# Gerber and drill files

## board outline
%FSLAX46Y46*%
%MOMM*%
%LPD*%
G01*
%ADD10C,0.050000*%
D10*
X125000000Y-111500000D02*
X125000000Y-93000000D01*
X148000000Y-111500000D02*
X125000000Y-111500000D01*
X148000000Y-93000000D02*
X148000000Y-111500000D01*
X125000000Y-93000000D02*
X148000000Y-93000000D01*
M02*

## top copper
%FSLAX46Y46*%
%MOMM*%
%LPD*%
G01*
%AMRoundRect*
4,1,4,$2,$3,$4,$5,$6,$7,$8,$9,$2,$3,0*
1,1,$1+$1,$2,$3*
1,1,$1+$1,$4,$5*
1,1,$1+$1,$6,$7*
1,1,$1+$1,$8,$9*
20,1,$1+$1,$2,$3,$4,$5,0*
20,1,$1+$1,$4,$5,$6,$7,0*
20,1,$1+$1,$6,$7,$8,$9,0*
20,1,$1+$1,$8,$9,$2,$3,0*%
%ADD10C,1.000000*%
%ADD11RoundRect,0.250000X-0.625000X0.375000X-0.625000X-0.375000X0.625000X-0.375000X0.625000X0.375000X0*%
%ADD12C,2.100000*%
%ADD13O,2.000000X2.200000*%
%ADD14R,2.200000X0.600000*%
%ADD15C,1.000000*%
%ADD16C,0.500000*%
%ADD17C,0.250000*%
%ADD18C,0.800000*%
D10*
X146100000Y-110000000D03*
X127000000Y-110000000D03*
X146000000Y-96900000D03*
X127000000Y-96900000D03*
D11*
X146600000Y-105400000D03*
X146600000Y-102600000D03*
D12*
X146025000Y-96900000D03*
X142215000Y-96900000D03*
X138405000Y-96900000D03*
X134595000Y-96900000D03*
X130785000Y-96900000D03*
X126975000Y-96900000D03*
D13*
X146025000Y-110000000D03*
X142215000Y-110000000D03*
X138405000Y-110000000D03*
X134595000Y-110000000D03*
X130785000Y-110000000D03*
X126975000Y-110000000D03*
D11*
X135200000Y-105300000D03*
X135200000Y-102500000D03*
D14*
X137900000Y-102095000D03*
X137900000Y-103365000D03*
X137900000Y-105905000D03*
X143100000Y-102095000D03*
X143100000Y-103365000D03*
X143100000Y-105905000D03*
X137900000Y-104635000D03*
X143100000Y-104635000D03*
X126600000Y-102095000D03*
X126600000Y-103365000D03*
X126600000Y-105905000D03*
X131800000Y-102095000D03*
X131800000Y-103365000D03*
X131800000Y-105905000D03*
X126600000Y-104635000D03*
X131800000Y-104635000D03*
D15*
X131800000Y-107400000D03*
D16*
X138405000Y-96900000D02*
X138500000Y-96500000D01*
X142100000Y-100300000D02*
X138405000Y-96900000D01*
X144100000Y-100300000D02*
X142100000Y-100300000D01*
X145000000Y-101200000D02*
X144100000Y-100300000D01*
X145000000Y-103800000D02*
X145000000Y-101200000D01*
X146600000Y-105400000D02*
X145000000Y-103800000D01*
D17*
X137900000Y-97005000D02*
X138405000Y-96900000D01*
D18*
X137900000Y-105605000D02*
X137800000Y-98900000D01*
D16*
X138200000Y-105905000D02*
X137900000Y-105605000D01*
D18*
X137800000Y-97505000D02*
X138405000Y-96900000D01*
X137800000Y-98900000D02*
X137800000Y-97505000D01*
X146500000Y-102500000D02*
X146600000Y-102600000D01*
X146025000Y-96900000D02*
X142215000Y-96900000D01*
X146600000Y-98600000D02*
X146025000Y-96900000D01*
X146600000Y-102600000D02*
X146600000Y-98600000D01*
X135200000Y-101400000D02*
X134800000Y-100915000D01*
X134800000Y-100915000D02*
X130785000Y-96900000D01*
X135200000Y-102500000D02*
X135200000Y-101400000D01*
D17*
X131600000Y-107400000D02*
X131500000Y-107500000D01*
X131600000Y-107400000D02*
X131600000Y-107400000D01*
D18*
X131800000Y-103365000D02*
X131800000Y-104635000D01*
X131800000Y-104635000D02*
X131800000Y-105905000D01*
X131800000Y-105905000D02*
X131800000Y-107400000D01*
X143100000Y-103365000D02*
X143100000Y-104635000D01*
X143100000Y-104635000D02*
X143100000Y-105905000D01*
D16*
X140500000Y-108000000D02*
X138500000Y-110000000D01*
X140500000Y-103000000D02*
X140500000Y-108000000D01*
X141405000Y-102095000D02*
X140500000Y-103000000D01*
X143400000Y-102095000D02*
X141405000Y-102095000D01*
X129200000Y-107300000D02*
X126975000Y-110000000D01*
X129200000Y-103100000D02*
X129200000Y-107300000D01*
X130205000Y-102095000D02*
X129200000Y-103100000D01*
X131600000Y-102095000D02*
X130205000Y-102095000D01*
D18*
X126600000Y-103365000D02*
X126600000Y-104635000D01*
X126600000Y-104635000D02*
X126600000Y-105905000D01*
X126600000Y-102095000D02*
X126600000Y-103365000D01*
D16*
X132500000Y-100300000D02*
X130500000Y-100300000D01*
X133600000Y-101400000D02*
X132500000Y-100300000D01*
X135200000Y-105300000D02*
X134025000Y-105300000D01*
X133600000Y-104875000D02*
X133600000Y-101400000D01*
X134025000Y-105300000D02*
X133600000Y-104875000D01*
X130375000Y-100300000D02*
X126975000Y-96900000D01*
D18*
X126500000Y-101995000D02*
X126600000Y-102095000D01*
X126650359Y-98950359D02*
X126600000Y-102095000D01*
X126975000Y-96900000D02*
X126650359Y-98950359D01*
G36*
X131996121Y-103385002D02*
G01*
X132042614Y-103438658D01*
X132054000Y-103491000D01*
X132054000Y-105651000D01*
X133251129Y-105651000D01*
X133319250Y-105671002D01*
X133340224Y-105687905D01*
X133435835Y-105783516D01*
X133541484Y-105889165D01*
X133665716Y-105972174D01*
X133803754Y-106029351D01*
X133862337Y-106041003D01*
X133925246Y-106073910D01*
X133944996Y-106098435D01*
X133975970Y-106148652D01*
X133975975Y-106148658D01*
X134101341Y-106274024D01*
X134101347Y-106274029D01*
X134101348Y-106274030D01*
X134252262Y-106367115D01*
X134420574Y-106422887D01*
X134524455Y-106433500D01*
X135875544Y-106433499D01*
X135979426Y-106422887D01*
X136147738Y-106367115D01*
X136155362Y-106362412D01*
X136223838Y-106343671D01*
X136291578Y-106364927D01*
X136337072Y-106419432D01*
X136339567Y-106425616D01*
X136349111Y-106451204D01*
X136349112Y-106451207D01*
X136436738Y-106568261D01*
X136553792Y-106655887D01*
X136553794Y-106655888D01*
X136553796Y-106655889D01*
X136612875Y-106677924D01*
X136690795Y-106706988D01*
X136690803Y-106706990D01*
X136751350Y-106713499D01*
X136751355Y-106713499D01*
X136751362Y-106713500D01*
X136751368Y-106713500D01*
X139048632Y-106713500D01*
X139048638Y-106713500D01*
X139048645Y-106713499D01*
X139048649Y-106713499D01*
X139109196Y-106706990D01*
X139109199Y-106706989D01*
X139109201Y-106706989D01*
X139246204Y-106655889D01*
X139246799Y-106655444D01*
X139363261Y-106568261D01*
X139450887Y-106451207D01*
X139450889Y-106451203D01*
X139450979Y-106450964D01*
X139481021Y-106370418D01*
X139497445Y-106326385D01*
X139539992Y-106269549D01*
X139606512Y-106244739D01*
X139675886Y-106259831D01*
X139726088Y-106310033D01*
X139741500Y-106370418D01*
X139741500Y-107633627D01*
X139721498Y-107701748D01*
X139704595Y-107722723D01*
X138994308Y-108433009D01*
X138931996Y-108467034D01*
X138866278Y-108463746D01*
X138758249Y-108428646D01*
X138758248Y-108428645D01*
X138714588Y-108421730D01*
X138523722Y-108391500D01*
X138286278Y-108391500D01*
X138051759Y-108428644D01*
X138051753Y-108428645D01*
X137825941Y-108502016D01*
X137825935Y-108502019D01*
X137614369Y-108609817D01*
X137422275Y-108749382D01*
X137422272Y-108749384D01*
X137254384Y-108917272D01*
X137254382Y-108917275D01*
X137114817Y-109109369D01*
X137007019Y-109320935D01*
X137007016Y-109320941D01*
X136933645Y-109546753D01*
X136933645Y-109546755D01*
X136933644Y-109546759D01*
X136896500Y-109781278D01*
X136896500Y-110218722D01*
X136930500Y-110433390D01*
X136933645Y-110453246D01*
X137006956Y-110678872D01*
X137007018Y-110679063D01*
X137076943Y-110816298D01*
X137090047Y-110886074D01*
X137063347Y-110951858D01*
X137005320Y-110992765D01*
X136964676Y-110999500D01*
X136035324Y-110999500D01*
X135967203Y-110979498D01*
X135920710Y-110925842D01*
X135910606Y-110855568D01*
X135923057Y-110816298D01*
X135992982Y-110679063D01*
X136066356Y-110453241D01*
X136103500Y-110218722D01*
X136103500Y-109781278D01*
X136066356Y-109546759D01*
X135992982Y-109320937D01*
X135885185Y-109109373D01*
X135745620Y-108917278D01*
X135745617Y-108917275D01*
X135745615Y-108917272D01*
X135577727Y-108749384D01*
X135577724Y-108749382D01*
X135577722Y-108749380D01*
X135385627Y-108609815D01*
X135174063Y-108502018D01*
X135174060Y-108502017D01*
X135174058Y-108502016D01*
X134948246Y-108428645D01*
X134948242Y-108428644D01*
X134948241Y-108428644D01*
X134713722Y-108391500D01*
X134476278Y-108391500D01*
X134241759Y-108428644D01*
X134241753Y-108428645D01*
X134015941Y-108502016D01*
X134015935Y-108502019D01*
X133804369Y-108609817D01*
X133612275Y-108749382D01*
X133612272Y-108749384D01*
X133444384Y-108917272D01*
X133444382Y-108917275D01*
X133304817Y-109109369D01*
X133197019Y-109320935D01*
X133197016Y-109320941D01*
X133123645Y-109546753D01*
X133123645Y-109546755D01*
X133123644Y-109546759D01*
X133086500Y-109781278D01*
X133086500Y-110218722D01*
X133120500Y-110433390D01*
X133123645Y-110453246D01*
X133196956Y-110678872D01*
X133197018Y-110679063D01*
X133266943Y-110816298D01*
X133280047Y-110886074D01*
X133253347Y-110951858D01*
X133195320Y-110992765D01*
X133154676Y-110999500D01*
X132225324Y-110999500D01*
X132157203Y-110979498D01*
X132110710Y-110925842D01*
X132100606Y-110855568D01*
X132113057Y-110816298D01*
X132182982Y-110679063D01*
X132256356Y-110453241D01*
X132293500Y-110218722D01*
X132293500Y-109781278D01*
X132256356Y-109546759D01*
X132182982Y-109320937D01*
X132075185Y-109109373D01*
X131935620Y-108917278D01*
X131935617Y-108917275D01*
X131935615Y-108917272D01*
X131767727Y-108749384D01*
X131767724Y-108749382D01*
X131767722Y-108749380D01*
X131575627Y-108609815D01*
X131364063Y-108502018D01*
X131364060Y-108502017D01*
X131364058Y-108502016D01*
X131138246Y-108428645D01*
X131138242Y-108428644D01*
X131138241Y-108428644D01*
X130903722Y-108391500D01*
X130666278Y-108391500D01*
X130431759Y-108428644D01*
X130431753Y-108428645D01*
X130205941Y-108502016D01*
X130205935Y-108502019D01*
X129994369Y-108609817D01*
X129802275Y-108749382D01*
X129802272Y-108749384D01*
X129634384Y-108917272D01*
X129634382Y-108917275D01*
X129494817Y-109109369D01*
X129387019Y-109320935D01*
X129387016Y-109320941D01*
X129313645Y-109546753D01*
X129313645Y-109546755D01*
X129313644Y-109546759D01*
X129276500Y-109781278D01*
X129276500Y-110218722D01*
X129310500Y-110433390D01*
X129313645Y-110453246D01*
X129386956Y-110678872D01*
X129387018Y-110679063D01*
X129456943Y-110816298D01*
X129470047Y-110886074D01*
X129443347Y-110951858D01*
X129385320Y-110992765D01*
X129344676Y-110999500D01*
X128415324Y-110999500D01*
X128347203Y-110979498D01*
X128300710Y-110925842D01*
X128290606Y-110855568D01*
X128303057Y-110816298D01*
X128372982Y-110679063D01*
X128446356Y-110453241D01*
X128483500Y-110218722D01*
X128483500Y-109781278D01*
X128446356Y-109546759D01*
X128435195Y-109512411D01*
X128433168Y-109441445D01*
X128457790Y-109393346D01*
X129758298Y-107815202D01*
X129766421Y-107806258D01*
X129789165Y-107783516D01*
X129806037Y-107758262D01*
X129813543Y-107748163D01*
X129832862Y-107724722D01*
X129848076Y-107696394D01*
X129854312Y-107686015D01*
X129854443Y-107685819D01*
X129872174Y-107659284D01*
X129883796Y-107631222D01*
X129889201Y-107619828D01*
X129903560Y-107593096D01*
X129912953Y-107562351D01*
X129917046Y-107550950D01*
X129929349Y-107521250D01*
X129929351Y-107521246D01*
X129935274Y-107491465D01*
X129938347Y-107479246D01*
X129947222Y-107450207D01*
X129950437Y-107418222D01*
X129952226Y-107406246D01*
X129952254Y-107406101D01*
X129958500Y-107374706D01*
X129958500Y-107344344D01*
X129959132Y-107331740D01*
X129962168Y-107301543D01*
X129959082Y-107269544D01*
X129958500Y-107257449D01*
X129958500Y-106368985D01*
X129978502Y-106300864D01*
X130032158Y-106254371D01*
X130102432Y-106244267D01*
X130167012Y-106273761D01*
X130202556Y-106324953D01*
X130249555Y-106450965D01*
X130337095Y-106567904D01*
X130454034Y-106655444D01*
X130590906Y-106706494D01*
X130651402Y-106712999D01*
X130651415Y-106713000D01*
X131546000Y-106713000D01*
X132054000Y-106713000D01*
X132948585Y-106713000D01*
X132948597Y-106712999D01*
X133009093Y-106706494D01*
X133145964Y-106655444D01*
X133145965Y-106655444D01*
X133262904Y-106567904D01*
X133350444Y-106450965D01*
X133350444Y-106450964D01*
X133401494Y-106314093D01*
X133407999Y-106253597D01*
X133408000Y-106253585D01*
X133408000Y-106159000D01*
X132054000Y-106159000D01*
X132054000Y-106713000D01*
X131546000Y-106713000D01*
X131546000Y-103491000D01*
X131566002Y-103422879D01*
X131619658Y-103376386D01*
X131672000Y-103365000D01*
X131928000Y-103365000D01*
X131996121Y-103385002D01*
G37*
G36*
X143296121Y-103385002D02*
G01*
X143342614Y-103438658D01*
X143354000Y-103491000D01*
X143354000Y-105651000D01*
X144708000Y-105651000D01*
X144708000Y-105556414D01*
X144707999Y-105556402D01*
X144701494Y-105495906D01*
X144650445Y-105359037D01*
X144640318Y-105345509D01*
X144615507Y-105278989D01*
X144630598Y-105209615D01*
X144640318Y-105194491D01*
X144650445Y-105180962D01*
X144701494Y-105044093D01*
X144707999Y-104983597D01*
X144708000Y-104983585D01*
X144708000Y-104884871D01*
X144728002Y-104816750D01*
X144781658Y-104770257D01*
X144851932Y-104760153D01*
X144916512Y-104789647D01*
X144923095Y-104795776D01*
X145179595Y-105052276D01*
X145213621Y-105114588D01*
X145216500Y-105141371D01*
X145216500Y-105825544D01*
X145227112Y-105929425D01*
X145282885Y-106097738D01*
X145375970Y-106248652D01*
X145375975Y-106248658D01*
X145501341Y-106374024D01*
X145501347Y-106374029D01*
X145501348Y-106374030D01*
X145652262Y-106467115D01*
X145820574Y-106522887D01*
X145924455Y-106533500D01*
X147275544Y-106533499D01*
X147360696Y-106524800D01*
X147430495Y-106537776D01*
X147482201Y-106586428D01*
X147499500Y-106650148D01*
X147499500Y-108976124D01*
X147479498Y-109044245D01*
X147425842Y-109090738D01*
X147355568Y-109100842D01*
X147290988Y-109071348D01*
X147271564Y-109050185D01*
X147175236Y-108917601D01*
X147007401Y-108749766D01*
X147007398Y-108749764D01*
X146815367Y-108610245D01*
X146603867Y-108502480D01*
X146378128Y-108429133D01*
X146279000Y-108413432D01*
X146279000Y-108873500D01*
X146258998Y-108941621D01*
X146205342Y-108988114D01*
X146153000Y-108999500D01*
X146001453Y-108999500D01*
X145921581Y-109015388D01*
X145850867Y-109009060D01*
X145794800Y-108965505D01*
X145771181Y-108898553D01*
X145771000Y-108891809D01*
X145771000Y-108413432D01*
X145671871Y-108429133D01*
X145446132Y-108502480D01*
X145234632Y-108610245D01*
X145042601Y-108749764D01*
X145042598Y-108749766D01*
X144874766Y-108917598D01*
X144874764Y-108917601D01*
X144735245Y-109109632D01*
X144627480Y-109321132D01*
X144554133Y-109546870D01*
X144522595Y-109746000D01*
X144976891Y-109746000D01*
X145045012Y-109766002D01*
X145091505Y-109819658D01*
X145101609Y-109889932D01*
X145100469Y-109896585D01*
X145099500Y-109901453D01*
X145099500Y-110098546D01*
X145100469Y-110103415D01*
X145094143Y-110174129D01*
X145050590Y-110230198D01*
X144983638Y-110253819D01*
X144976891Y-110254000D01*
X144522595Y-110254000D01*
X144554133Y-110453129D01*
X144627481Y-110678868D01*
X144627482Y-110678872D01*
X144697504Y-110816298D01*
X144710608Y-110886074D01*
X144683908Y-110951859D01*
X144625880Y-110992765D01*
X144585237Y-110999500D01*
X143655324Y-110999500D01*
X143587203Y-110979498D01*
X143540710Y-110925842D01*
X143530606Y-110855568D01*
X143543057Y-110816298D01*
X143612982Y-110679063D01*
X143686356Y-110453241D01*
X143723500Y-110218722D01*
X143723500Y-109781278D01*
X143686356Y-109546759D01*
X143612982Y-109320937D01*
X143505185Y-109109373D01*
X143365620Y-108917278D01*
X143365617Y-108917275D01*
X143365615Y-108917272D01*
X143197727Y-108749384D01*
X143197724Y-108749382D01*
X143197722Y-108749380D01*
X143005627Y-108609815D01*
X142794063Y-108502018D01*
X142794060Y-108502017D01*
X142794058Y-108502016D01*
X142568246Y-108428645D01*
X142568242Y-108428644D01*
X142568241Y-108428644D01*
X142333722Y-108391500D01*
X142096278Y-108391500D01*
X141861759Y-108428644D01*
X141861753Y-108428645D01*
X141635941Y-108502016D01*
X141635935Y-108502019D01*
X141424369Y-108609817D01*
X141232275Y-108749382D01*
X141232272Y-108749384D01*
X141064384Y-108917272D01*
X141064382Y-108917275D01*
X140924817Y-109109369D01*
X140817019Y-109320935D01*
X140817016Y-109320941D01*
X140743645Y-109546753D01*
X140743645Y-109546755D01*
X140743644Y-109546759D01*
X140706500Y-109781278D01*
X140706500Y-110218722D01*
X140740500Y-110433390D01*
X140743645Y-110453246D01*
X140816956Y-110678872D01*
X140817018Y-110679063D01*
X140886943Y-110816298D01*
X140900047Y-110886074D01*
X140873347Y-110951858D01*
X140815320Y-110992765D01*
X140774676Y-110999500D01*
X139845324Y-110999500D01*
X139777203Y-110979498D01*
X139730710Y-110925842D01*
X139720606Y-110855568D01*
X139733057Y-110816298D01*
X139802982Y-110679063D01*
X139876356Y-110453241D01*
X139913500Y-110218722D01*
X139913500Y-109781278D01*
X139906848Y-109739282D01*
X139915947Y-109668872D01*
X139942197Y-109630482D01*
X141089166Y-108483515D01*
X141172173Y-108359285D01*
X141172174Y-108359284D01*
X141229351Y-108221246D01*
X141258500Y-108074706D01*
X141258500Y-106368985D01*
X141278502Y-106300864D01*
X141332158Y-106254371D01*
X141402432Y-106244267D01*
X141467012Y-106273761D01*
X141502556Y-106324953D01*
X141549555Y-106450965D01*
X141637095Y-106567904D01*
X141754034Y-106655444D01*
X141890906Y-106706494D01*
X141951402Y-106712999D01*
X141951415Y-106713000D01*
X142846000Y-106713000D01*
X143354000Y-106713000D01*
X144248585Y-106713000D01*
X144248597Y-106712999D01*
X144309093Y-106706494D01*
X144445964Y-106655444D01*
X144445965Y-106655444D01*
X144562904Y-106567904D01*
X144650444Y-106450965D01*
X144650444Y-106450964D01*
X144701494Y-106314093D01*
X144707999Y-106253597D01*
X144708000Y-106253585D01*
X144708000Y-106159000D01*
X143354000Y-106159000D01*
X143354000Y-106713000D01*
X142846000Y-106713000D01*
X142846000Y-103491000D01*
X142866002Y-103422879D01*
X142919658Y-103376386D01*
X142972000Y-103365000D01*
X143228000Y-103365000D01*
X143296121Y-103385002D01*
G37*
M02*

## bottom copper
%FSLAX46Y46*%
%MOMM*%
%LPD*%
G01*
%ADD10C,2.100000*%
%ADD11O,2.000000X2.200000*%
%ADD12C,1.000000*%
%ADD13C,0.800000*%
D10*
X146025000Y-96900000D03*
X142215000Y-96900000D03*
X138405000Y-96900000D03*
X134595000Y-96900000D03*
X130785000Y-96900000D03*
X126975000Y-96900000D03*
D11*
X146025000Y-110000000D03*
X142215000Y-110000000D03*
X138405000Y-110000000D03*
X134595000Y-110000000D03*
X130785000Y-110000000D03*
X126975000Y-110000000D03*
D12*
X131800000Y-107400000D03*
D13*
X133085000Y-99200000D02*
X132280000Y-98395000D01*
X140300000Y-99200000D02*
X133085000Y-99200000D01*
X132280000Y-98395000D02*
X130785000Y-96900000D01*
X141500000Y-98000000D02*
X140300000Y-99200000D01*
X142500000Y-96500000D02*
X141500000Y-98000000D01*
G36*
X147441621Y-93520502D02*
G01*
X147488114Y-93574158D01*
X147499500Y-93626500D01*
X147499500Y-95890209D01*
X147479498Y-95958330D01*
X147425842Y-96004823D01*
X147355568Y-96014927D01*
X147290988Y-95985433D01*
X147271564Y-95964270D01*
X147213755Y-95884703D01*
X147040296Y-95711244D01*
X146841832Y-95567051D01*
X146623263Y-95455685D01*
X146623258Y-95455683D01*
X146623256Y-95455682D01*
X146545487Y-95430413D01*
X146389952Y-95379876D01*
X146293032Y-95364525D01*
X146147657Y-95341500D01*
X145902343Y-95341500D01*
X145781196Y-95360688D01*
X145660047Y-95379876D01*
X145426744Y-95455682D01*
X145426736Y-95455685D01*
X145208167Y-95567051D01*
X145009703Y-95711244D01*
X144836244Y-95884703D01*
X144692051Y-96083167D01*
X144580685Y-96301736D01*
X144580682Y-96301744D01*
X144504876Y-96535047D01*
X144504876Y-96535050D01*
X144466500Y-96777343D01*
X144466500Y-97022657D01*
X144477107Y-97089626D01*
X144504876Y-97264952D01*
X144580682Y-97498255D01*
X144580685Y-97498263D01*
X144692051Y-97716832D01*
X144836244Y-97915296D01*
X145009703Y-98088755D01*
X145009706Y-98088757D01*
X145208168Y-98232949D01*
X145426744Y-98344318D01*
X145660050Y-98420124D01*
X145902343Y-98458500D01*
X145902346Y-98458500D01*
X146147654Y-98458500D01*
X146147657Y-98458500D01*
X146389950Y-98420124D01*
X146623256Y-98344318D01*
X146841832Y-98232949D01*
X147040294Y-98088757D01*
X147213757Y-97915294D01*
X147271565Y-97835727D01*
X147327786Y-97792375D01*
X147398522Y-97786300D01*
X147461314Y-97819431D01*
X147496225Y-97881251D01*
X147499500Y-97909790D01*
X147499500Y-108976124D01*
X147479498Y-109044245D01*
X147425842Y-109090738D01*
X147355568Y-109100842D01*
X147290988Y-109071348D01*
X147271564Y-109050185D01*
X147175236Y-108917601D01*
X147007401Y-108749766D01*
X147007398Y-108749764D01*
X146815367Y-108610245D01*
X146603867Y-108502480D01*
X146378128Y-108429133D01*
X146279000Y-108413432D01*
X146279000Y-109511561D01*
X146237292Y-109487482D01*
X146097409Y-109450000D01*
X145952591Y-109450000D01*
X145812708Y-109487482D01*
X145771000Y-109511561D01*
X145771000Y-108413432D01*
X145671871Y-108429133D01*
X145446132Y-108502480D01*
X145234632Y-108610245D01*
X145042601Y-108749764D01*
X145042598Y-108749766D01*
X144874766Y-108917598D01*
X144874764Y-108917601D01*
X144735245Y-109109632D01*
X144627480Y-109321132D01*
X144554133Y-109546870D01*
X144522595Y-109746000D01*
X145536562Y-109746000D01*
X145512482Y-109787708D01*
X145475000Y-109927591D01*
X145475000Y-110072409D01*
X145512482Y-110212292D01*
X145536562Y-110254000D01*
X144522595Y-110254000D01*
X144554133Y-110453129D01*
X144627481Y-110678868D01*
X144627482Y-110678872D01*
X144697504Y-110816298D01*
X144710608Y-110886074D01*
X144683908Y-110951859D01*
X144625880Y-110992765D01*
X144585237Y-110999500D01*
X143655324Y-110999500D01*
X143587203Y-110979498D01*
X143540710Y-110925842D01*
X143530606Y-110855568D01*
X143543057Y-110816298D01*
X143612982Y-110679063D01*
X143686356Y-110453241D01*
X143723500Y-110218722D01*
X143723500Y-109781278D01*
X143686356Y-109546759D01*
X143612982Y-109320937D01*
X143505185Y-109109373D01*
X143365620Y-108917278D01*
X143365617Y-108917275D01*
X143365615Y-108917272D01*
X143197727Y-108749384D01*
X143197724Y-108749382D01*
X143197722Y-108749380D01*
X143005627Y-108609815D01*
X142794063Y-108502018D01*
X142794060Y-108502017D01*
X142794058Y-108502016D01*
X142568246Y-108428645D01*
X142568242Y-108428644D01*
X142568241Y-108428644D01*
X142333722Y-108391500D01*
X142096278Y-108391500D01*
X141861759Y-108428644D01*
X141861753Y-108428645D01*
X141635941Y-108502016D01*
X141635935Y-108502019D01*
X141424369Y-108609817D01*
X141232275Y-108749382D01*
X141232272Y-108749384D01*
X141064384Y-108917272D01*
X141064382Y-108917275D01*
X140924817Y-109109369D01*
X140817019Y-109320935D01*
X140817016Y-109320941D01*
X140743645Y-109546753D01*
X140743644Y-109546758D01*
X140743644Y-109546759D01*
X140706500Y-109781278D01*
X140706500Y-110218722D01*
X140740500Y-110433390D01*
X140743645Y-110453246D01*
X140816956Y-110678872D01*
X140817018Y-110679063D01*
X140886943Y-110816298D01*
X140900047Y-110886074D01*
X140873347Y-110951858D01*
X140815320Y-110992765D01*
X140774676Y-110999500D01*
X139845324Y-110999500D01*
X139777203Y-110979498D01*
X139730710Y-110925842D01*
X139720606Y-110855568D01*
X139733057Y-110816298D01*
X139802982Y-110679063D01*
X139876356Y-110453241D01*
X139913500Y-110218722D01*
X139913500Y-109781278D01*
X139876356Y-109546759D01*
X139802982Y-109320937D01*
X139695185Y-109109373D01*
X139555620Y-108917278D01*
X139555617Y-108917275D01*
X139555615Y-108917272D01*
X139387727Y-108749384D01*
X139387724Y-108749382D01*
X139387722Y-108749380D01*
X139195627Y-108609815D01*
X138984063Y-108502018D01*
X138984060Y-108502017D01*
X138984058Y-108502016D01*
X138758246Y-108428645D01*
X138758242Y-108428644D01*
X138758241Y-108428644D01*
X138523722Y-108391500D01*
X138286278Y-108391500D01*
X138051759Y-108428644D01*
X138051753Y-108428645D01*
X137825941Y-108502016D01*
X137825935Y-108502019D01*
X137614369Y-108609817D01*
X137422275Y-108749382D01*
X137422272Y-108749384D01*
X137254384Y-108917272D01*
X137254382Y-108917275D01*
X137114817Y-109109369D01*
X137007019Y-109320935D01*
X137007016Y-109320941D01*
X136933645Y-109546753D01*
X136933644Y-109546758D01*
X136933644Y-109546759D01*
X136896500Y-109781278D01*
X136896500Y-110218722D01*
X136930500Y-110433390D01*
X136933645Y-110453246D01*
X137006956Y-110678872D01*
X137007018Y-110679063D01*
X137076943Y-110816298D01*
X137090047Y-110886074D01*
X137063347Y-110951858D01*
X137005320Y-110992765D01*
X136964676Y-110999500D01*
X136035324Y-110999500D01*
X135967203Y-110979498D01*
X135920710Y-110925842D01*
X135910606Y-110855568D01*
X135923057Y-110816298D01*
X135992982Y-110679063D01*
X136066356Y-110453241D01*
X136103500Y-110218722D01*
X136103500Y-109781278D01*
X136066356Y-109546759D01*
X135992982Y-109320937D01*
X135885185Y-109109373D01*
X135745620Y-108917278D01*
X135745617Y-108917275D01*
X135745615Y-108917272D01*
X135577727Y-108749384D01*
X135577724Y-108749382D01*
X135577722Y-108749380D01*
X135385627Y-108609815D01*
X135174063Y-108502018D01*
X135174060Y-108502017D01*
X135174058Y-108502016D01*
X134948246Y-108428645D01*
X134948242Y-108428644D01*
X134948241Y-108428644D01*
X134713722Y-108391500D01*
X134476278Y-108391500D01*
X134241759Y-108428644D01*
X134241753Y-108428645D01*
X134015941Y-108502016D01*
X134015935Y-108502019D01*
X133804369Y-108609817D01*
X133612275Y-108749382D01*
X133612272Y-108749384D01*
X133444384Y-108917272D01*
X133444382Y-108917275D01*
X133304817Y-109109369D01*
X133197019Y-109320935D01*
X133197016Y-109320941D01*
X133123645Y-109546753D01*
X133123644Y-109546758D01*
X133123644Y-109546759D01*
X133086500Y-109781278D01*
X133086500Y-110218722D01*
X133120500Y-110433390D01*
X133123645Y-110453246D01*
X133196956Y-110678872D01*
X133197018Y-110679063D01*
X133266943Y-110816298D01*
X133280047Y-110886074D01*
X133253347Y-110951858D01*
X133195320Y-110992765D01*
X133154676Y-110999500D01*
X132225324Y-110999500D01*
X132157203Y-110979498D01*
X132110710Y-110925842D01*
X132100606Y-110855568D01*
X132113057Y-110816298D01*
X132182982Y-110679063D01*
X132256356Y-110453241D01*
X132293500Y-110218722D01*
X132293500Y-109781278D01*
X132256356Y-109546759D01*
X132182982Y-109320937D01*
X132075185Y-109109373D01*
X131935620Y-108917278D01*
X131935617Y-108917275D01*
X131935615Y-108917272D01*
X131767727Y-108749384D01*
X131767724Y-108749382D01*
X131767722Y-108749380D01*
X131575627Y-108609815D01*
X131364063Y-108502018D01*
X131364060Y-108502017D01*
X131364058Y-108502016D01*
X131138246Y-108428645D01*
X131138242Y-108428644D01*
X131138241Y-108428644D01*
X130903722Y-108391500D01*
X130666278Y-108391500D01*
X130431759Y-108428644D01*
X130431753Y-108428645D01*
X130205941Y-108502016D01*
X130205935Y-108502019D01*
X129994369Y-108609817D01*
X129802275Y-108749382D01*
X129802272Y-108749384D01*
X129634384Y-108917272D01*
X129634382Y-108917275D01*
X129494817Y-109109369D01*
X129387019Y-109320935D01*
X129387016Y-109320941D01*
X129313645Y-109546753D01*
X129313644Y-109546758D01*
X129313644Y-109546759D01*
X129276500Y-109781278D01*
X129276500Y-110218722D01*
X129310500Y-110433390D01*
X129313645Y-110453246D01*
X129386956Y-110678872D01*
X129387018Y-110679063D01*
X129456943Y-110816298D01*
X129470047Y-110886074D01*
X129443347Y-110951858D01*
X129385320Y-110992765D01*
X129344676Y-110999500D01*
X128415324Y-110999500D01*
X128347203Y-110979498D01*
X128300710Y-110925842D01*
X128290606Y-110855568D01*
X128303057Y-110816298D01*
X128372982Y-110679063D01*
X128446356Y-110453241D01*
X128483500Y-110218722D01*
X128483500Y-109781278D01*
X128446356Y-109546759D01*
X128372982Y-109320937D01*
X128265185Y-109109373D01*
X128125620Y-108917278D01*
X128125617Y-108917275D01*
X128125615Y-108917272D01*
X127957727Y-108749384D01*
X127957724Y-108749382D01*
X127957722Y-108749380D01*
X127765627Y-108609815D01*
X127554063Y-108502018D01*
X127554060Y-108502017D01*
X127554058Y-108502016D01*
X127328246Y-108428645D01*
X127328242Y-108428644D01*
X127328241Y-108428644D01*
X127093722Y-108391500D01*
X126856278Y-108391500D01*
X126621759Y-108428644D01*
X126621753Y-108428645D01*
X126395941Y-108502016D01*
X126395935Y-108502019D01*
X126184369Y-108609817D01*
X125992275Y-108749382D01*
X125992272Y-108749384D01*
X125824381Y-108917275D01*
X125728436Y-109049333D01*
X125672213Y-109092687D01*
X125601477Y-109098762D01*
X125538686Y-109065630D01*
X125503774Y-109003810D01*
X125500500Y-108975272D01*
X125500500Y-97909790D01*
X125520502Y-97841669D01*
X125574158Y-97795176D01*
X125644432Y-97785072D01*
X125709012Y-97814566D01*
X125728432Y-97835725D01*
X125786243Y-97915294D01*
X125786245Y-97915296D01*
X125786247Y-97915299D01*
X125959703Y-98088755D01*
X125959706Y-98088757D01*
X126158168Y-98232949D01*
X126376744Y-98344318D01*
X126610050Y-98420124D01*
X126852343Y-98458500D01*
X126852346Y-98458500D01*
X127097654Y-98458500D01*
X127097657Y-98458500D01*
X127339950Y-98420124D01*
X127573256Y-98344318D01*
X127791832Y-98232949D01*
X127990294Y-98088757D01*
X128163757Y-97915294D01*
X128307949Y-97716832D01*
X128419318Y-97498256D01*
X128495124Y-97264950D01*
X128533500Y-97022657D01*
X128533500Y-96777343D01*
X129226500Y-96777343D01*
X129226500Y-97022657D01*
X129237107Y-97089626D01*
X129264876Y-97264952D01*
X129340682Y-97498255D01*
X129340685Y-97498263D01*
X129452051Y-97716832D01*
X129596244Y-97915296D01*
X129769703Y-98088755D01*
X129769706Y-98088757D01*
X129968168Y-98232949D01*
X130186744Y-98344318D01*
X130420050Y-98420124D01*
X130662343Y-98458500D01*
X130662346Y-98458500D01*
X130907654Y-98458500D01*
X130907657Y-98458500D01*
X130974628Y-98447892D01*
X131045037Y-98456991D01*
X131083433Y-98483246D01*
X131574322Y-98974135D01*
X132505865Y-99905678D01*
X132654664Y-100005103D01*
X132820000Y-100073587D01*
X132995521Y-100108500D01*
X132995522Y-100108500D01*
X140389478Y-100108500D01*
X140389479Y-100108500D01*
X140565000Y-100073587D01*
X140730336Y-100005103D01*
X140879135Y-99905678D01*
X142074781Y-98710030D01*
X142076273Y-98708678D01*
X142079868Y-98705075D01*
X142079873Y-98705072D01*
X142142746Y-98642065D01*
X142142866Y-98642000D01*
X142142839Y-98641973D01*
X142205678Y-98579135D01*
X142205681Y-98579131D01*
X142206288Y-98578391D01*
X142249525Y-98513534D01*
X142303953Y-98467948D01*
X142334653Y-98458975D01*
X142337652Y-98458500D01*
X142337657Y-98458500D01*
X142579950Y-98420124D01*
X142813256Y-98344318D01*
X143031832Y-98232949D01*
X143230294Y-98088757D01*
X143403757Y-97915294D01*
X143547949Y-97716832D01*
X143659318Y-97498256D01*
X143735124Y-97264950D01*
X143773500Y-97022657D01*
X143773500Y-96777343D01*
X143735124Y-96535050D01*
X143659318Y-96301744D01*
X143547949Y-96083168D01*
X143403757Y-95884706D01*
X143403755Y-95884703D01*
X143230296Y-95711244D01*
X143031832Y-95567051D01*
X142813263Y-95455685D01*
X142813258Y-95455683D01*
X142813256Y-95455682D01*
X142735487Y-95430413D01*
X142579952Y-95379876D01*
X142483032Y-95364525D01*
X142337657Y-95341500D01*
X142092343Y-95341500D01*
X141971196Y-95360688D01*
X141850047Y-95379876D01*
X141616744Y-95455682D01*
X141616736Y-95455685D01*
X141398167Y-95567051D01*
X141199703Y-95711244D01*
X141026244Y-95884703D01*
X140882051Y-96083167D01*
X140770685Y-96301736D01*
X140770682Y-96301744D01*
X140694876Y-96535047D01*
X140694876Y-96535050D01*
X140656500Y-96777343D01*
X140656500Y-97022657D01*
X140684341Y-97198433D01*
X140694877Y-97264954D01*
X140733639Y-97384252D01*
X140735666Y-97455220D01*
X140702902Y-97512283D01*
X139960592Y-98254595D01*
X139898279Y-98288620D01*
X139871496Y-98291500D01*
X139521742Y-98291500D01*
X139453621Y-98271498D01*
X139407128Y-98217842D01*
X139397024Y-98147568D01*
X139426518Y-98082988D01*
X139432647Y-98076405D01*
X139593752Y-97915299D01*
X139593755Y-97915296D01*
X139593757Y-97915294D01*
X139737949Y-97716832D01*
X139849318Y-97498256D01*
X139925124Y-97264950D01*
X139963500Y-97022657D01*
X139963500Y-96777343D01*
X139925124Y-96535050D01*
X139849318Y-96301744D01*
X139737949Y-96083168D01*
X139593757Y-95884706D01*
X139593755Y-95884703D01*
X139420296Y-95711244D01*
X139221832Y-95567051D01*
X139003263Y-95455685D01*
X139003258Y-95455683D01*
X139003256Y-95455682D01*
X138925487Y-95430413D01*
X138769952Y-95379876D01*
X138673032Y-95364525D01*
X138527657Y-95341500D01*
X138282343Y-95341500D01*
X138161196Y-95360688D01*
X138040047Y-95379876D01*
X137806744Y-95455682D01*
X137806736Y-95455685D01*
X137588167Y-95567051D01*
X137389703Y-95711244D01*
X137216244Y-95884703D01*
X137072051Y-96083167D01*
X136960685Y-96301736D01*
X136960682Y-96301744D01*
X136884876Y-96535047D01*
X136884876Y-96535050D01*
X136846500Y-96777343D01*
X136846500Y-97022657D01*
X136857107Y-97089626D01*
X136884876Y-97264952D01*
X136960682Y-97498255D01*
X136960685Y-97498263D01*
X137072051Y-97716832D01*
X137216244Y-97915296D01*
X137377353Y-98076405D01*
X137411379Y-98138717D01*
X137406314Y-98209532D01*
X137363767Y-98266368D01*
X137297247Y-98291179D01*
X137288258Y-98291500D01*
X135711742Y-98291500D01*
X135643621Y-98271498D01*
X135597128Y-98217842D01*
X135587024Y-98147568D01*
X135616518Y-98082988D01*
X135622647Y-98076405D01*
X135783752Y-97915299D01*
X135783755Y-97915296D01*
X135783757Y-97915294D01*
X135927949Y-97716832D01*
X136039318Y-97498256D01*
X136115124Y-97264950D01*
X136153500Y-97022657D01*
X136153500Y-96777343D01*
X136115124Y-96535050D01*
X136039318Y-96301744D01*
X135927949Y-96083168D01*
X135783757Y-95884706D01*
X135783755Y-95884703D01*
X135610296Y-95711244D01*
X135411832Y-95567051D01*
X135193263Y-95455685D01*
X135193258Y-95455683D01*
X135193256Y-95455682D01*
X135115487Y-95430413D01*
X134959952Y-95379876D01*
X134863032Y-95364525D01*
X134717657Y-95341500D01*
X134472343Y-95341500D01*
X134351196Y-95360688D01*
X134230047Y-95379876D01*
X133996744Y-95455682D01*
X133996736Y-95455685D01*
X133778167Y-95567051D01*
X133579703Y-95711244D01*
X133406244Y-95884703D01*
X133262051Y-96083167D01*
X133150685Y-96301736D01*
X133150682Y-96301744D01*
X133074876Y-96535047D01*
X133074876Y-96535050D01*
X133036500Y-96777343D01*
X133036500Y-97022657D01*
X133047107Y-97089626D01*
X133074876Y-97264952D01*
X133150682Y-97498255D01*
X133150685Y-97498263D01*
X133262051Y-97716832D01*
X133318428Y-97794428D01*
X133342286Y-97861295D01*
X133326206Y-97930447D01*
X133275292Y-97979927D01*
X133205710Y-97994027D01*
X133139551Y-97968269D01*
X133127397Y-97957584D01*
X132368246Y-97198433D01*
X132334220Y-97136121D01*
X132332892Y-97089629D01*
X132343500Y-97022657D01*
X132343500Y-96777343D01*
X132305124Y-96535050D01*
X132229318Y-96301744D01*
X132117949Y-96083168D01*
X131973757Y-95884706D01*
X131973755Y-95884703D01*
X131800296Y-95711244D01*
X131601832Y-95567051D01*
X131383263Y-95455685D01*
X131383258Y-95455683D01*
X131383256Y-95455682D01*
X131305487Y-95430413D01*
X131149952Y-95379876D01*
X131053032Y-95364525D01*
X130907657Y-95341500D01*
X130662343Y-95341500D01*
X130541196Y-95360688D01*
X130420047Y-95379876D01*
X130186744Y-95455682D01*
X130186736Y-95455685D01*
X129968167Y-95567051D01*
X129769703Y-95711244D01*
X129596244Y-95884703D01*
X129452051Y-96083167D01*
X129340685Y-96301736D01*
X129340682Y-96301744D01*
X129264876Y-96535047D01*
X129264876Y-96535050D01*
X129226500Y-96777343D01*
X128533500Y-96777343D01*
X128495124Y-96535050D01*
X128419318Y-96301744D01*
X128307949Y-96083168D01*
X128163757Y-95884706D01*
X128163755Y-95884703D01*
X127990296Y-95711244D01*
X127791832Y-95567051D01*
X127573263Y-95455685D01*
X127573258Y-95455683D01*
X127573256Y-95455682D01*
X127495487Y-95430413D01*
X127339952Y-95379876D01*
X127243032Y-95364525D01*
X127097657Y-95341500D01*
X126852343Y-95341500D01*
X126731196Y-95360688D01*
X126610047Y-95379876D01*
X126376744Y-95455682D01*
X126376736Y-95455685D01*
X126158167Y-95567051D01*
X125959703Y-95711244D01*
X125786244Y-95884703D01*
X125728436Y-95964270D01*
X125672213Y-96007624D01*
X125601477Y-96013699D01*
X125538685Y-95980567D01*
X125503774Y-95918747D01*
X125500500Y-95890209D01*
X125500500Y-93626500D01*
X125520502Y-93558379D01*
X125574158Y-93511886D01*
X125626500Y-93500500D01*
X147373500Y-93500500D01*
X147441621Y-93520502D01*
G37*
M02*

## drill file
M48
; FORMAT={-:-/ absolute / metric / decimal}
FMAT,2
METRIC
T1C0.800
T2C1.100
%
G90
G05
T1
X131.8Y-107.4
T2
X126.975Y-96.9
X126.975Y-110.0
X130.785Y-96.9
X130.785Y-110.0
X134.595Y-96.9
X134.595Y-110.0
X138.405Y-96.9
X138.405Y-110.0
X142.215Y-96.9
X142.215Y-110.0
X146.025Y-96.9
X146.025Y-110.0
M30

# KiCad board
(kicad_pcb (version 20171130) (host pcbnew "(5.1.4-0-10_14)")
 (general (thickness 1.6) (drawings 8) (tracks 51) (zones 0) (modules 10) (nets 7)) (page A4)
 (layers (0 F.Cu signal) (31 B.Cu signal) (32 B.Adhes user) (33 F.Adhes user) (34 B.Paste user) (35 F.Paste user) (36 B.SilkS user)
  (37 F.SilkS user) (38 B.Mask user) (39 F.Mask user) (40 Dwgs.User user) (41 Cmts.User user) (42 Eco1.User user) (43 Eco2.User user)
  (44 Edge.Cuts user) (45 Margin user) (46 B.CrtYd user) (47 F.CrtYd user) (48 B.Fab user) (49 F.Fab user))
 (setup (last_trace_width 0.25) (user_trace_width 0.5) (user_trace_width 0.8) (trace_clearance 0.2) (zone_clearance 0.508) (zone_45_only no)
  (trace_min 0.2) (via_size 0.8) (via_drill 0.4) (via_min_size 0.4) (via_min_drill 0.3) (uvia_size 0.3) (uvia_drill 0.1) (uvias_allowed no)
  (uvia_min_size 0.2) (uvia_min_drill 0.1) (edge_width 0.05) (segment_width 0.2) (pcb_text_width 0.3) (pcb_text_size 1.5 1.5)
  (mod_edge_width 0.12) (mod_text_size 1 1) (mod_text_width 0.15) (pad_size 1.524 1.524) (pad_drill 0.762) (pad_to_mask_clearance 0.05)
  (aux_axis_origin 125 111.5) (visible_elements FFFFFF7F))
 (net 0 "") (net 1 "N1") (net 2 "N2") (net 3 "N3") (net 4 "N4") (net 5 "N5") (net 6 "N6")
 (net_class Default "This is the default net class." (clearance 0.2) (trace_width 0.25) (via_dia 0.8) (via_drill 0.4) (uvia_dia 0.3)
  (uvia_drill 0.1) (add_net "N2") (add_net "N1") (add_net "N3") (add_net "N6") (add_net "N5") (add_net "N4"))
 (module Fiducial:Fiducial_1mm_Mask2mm (layer F.Cu) (at 146.1 110)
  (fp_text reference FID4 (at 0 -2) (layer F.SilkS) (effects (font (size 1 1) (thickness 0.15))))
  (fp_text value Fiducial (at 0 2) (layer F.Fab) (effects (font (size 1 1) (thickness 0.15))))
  (pad "" smd circle (at 0 0) (size 1 1) (layers F.Cu F.Mask) (solder_mask_margin 0.5) (clearance 0.5)))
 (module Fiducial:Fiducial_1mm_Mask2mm (layer F.Cu) (at 127 110)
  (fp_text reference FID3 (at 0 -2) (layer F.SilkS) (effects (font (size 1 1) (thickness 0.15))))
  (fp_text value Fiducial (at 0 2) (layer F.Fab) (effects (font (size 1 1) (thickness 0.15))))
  (pad "" smd circle (at 0 0) (size 1 1) (layers F.Cu F.Mask) (solder_mask_margin 0.5) (clearance 0.5)))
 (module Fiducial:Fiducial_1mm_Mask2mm (layer F.Cu) (at 146 96.9)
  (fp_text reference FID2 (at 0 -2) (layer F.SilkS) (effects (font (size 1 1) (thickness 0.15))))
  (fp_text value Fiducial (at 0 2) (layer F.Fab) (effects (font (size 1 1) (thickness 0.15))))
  (pad "" smd circle (at 0 0) (size 1 1) (layers F.Cu F.Mask) (solder_mask_margin 0.5) (clearance 0.5)))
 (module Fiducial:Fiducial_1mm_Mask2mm (layer F.Cu) (at 127 96.9)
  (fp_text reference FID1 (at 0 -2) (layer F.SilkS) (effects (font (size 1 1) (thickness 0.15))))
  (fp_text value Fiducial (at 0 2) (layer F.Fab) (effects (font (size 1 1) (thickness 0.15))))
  (pad "" smd circle (at 0 0) (size 1 1) (layers F.Cu F.Mask) (solder_mask_margin 0.5) (clearance 0.5)))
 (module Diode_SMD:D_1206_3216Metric (layer F.Cu) (at 146.6 104 270)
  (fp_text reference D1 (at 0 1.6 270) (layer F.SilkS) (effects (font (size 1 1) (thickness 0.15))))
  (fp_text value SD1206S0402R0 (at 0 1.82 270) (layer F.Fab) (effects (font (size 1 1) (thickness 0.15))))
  (pad 2 smd roundrect (at 1.4 0 270) (size 1.25 1.75) (layers F.Cu F.Paste F.Mask) (roundrect_rratio 0.2) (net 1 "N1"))
  (pad 1 smd roundrect (at -1.4 0 270) (size 1.25 1.75) (layers F.Cu F.Paste F.Mask) (roundrect_rratio 0.2) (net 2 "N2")))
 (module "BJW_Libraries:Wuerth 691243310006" (layer F.Cu) (at 136.5 96.9)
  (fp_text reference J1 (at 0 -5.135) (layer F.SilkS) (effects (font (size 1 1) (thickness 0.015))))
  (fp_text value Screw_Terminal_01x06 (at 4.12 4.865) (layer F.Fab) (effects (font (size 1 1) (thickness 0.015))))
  (pad 6 thru_hole circle (at 9.525 0) (size 2.1 2.1) (drill 1.1) (layers *.Cu *.Mask) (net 2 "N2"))
  (pad 5 thru_hole circle (at 5.715 0) (size 2.1 2.1) (drill 1.1) (layers *.Cu *.Mask) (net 2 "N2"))
  (pad 4 thru_hole circle (at 1.905 0) (size 2.1 2.1) (drill 1.1) (layers *.Cu *.Mask) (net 1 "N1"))
  (pad 3 thru_hole circle (at -1.905 0) (size 2.1 2.1) (drill 1.1) (layers *.Cu *.Mask))
  (pad 2 thru_hole circle (at -5.715 0) (size 2.1 2.1) (drill 1.1) (layers *.Cu *.Mask) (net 2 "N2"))
  (pad 1 thru_hole circle (at -9.525 0) (size 2.1 2.1) (drill 1.1) (layers *.Cu *.Mask) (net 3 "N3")))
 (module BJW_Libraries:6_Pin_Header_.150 (layer F.Cu) (at 136.5 110)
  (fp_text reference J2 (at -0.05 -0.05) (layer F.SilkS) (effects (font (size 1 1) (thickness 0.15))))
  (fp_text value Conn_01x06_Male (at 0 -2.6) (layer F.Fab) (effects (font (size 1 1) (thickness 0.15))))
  (pad 6 thru_hole oval (at 9.525 0) (size 2 2.2) (drill 1.1) (layers *.Cu *.Mask) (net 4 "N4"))
  (pad 5 thru_hole oval (at 5.715 0) (size 2 2.2) (drill 1.1) (layers *.Cu *.Mask))
  (pad 4 thru_hole oval (at 1.905 0) (size 2 2.2) (drill 1.1) (layers *.Cu *.Mask) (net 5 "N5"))
  (pad 3 thru_hole oval (at -1.905 0) (size 2 2.2) (drill 1.1) (layers *.Cu *.Mask))
  (pad 2 thru_hole oval (at -5.715 0) (size 2 2.2) (drill 1.1) (layers *.Cu *.Mask))
  (pad 1 thru_hole oval (at -9.525 0) (size 2 2.2) (drill 1.1) (layers *.Cu *.Mask) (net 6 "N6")))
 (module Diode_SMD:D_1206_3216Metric (layer F.Cu) (at 135.2 103.9 270)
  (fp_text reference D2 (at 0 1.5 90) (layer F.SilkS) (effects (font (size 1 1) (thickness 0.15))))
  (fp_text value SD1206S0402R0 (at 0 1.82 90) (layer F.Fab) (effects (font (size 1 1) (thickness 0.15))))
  (pad 2 smd roundrect (at 1.4 0 270) (size 1.25 1.75) (layers F.Cu F.Paste F.Mask) (roundrect_rratio 0.2) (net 3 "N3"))
  (pad 1 smd roundrect (at -1.4 0 270) (size 1.25 1.75) (layers F.Cu F.Paste F.Mask) (roundrect_rratio 0.2) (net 2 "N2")))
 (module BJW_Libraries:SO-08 (layer F.Cu) (at 140.5 104 90)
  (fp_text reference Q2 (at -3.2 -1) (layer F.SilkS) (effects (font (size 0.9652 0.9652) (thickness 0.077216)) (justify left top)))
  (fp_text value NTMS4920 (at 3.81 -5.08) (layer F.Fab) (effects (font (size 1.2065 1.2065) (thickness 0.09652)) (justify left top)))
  (pad 5 smd rect (at 1.905 -2.6 90) (size 0.6 2.2) (layers F.Cu F.Paste F.Mask) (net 1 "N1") (solder_mask_margin 0.1016))
  (pad 6 smd rect (at 0.635 -2.6 90) (size 0.6 2.2) (layers F.Cu F.Paste F.Mask) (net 1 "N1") (solder_mask_margin 0.1016))
  (pad 8 smd rect (at -1.905 -2.6 90) (size 0.6 2.2) (layers F.Cu F.Paste F.Mask) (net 1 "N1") (solder_mask_margin 0.1016))
  (pad 4 smd rect (at 1.905 2.6 90) (size 0.6 2.2) (layers F.Cu F.Paste F.Mask) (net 5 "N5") (solder_mask_margin 0.1016))
  (pad 3 smd rect (at 0.635 2.6 90) (size 0.6 2.2) (layers F.Cu F.Paste F.Mask) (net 4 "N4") (solder_mask_margin 0.1016))
  (pad 1 smd rect (at -1.905 2.6 90) (size 0.6 2.2) (layers F.Cu F.Paste F.Mask) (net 4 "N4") (solder_mask_margin 0.1016))
  (pad 7 smd rect (at -0.635 -2.6 90) (size 0.6 2.2) (layers F.Cu F.Paste F.Mask) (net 1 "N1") (solder_mask_margin 0.1016))
  (pad 2 smd rect (at -0.635 2.6 90) (size 0.6 2.2) (layers F.Cu F.Paste F.Mask) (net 4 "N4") (solder_mask_margin 0.1016)))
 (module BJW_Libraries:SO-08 (layer F.Cu) (at 129.2 104 90)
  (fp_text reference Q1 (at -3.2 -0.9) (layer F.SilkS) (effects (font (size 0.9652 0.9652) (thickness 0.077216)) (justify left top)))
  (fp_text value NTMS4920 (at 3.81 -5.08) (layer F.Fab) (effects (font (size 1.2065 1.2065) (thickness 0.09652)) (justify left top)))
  (pad 5 smd rect (at 1.905 -2.6 90) (size 0.6 2.2) (layers F.Cu F.Paste F.Mask) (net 3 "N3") (solder_mask_margin 0.1016))
  (pad 6 smd rect (at 0.635 -2.6 90) (size 0.6 2.2) (layers F.Cu F.Paste F.Mask) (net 3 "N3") (solder_mask_margin 0.1016))
  (pad 8 smd rect (at -1.905 -2.6 90) (size 0.6 2.2) (layers F.Cu F.Paste F.Mask) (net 3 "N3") (solder_mask_margin 0.1016))
  (pad 4 smd rect (at 1.905 2.6 90) (size 0.6 2.2) (layers F.Cu F.Paste F.Mask) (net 6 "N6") (solder_mask_margin 0.1016))
  (pad 3 smd rect (at 0.635 2.6 90) (size 0.6 2.2) (layers F.Cu F.Paste F.Mask) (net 4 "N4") (solder_mask_margin 0.1016))
  (pad 1 smd rect (at -1.905 2.6 90) (size 0.6 2.2) (layers F.Cu F.Paste F.Mask) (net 4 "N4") (solder_mask_margin 0.1016))
  (pad 7 smd rect (at -0.635 -2.6 90) (size 0.6 2.2) (layers F.Cu F.Paste F.Mask) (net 3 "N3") (solder_mask_margin 0.1016))
  (pad 2 smd rect (at -0.635 2.6 90) (size 0.6 2.2) (layers F.Cu F.Paste F.Mask) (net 4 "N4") (solder_mask_margin 0.1016)))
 (gr_line (start 125 111.5) (end 125 93) (layer Edge.Cuts) (width 0.05))
 (gr_line (start 148 111.5) (end 125 111.5) (layer Edge.Cuts) (width 0.05))
 (gr_line (start 148 93) (end 148 111.5) (layer Edge.Cuts) (width 0.05))
 (gr_line (start 125 93) (end 148 93) (layer Edge.Cuts) (width 0.05))
 (segment (start 138.405 96.9) (end 138.5 96.5) (width 0.5) (layer F.Cu) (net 1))
 (segment (start 142.1 100.3) (end 138.405 96.9) (width 0.5) (layer F.Cu) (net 1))
 (segment (start 144.1 100.3) (end 142.1 100.3) (width 0.5) (layer F.Cu) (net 1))
 (segment (start 145 101.2) (end 144.1 100.3) (width 0.5) (layer F.Cu) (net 1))
 (segment (start 145 103.8) (end 145 101.2) (width 0.5) (layer F.Cu) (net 1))
 (segment (start 146.6 105.4) (end 145 103.8) (width 0.5) (layer F.Cu) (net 1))
 (segment (start 137.9 97.005) (end 138.405 96.9) (width 0.25) (layer F.Cu) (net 1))
 (segment (start 137.9 105.605) (end 137.8 98.9) (width 0.8) (layer F.Cu) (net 1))
 (segment (start 138.2 105.905) (end 137.9 105.605) (width 0.5) (layer F.Cu) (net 1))
 (segment (start 137.8 97.505) (end 138.405 96.9) (width 0.8) (layer F.Cu) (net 1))
 (segment (start 137.8 98.9) (end 137.8 97.505) (width 0.8) (layer F.Cu) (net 1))
 (segment (start 146.5 102.5) (end 146.6 102.6) (width 0.8) (layer F.Cu) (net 2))
 (segment (start 146.025 96.9) (end 142.215 96.9) (width 0.8) (layer F.Cu) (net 2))
 (segment (start 146.6 98.6) (end 146.025 96.9) (width 0.8) (layer F.Cu) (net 2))
 (segment (start 146.6 102.6) (end 146.6 98.6) (width 0.8) (layer F.Cu) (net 2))
 (segment (start 135.2 101.4) (end 134.8 100.915) (width 0.8) (layer F.Cu) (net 2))
 (segment (start 134.8 100.915) (end 130.785 96.9) (width 0.8) (layer F.Cu) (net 2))
 (segment (start 135.2 102.5) (end 135.2 101.4) (width 0.8) (layer F.Cu) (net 2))
 (segment (start 133.085 99.2) (end 132.28 98.395) (width 0.8) (layer B.Cu) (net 2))
 (segment (start 140.3 99.2) (end 133.085 99.2) (width 0.8) (layer B.Cu) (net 2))
 (segment (start 132.28 98.395) (end 130.785 96.9) (width 0.8) (layer B.Cu) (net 2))
 (segment (start 141.5 98) (end 140.3 99.2) (width 0.8) (layer B.Cu) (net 2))
 (segment (start 142.5 96.5) (end 141.5 98) (width 0.8) (layer B.Cu) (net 2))
 (via (at 131.8 107.4) (size 1) (drill 0.8) (layers F.Cu B.Cu) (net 4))
 (segment (start 131.6 107.4) (end 131.5 107.5) (width 0.25) (layer F.Cu) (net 4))
 (segment (start 131.6 107.4) (end 131.6 107.4) (width 0.25) (layer F.Cu) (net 4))
 (segment (start 131.8 103.365) (end 131.8 104.635) (width 0.8) (layer F.Cu) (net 4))
 (segment (start 131.8 104.635) (end 131.8 105.905) (width 0.8) (layer F.Cu) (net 4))
 (segment (start 131.8 105.905) (end 131.8 107.4) (width 0.8) (layer F.Cu) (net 4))
 (segment (start 143.1 103.365) (end 143.1 104.635) (width 0.8) (layer F.Cu) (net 4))
 (segment (start 143.1 104.635) (end 143.1 105.905) (width 0.8) (layer F.Cu) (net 4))
 (segment (start 140.5 108) (end 138.5 110) (width 0.5) (layer F.Cu) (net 5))
 (segment (start 140.5 103) (end 140.5 108) (width 0.5) (layer F.Cu) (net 5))
 (segment (start 141.405 102.095) (end 140.5 103) (width 0.5) (layer F.Cu) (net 5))
 (segment (start 143.4 102.095) (end 141.405 102.095) (width 0.5) (layer F.Cu) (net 5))
 (segment (start 129.2 107.3) (end 126.975 110) (width 0.5) (layer F.Cu) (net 6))
 (segment (start 129.2 103.1) (end 129.2 107.3) (width 0.5) (layer F.Cu) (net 6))
 (segment (start 130.205 102.095) (end 129.2 103.1) (width 0.5) (layer F.Cu) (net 6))
 (segment (start 131.6 102.095) (end 130.205 102.095) (width 0.5) (layer F.Cu) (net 6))
 (segment (start 126.6 103.365) (end 126.6 104.635) (width 0.8) (layer F.Cu) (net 3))
 (segment (start 126.6 104.635) (end 126.6 105.905) (width 0.8) (layer F.Cu) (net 3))
 (segment (start 126.6 102.095) (end 126.6 103.365) (width 0.8) (layer F.Cu) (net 3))
 (segment (start 132.5 100.3) (end 130.5 100.3) (width 0.5) (layer F.Cu) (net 3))
 (segment (start 133.6 101.4) (end 132.5 100.3) (width 0.5) (layer F.Cu) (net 3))
 (segment (start 135.2 105.3) (end 134.025 105.3) (width 0.5) (layer F.Cu) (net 3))
 (segment (start 133.6 104.875) (end 133.6 101.4) (width 0.5) (layer F.Cu) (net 3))
 (segment (start 134.025 105.3) (end 133.6 104.875) (width 0.5) (layer F.Cu) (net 3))
 (segment (start 130.375 100.3) (end 126.975 96.9) (width 0.5) (layer F.Cu) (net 3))
 (segment (start 126.5 101.995) (end 126.6 102.095) (width 0.8) (layer F.Cu) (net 3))
 (segment (start 126.650359 98.950359) (end 126.6 102.095) (width 0.8) (layer F.Cu) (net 3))
 (segment (start 126.975 96.9) (end 126.650359 98.950359) (width 0.8) (layer F.Cu) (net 3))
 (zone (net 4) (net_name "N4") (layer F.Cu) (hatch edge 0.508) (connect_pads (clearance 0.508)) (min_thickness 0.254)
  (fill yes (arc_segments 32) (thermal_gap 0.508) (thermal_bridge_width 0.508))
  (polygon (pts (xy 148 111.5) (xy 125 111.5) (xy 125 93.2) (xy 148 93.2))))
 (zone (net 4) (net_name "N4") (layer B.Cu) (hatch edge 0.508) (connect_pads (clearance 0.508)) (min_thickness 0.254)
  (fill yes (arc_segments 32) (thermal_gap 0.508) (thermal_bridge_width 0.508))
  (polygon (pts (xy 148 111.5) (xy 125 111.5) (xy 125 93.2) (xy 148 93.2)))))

